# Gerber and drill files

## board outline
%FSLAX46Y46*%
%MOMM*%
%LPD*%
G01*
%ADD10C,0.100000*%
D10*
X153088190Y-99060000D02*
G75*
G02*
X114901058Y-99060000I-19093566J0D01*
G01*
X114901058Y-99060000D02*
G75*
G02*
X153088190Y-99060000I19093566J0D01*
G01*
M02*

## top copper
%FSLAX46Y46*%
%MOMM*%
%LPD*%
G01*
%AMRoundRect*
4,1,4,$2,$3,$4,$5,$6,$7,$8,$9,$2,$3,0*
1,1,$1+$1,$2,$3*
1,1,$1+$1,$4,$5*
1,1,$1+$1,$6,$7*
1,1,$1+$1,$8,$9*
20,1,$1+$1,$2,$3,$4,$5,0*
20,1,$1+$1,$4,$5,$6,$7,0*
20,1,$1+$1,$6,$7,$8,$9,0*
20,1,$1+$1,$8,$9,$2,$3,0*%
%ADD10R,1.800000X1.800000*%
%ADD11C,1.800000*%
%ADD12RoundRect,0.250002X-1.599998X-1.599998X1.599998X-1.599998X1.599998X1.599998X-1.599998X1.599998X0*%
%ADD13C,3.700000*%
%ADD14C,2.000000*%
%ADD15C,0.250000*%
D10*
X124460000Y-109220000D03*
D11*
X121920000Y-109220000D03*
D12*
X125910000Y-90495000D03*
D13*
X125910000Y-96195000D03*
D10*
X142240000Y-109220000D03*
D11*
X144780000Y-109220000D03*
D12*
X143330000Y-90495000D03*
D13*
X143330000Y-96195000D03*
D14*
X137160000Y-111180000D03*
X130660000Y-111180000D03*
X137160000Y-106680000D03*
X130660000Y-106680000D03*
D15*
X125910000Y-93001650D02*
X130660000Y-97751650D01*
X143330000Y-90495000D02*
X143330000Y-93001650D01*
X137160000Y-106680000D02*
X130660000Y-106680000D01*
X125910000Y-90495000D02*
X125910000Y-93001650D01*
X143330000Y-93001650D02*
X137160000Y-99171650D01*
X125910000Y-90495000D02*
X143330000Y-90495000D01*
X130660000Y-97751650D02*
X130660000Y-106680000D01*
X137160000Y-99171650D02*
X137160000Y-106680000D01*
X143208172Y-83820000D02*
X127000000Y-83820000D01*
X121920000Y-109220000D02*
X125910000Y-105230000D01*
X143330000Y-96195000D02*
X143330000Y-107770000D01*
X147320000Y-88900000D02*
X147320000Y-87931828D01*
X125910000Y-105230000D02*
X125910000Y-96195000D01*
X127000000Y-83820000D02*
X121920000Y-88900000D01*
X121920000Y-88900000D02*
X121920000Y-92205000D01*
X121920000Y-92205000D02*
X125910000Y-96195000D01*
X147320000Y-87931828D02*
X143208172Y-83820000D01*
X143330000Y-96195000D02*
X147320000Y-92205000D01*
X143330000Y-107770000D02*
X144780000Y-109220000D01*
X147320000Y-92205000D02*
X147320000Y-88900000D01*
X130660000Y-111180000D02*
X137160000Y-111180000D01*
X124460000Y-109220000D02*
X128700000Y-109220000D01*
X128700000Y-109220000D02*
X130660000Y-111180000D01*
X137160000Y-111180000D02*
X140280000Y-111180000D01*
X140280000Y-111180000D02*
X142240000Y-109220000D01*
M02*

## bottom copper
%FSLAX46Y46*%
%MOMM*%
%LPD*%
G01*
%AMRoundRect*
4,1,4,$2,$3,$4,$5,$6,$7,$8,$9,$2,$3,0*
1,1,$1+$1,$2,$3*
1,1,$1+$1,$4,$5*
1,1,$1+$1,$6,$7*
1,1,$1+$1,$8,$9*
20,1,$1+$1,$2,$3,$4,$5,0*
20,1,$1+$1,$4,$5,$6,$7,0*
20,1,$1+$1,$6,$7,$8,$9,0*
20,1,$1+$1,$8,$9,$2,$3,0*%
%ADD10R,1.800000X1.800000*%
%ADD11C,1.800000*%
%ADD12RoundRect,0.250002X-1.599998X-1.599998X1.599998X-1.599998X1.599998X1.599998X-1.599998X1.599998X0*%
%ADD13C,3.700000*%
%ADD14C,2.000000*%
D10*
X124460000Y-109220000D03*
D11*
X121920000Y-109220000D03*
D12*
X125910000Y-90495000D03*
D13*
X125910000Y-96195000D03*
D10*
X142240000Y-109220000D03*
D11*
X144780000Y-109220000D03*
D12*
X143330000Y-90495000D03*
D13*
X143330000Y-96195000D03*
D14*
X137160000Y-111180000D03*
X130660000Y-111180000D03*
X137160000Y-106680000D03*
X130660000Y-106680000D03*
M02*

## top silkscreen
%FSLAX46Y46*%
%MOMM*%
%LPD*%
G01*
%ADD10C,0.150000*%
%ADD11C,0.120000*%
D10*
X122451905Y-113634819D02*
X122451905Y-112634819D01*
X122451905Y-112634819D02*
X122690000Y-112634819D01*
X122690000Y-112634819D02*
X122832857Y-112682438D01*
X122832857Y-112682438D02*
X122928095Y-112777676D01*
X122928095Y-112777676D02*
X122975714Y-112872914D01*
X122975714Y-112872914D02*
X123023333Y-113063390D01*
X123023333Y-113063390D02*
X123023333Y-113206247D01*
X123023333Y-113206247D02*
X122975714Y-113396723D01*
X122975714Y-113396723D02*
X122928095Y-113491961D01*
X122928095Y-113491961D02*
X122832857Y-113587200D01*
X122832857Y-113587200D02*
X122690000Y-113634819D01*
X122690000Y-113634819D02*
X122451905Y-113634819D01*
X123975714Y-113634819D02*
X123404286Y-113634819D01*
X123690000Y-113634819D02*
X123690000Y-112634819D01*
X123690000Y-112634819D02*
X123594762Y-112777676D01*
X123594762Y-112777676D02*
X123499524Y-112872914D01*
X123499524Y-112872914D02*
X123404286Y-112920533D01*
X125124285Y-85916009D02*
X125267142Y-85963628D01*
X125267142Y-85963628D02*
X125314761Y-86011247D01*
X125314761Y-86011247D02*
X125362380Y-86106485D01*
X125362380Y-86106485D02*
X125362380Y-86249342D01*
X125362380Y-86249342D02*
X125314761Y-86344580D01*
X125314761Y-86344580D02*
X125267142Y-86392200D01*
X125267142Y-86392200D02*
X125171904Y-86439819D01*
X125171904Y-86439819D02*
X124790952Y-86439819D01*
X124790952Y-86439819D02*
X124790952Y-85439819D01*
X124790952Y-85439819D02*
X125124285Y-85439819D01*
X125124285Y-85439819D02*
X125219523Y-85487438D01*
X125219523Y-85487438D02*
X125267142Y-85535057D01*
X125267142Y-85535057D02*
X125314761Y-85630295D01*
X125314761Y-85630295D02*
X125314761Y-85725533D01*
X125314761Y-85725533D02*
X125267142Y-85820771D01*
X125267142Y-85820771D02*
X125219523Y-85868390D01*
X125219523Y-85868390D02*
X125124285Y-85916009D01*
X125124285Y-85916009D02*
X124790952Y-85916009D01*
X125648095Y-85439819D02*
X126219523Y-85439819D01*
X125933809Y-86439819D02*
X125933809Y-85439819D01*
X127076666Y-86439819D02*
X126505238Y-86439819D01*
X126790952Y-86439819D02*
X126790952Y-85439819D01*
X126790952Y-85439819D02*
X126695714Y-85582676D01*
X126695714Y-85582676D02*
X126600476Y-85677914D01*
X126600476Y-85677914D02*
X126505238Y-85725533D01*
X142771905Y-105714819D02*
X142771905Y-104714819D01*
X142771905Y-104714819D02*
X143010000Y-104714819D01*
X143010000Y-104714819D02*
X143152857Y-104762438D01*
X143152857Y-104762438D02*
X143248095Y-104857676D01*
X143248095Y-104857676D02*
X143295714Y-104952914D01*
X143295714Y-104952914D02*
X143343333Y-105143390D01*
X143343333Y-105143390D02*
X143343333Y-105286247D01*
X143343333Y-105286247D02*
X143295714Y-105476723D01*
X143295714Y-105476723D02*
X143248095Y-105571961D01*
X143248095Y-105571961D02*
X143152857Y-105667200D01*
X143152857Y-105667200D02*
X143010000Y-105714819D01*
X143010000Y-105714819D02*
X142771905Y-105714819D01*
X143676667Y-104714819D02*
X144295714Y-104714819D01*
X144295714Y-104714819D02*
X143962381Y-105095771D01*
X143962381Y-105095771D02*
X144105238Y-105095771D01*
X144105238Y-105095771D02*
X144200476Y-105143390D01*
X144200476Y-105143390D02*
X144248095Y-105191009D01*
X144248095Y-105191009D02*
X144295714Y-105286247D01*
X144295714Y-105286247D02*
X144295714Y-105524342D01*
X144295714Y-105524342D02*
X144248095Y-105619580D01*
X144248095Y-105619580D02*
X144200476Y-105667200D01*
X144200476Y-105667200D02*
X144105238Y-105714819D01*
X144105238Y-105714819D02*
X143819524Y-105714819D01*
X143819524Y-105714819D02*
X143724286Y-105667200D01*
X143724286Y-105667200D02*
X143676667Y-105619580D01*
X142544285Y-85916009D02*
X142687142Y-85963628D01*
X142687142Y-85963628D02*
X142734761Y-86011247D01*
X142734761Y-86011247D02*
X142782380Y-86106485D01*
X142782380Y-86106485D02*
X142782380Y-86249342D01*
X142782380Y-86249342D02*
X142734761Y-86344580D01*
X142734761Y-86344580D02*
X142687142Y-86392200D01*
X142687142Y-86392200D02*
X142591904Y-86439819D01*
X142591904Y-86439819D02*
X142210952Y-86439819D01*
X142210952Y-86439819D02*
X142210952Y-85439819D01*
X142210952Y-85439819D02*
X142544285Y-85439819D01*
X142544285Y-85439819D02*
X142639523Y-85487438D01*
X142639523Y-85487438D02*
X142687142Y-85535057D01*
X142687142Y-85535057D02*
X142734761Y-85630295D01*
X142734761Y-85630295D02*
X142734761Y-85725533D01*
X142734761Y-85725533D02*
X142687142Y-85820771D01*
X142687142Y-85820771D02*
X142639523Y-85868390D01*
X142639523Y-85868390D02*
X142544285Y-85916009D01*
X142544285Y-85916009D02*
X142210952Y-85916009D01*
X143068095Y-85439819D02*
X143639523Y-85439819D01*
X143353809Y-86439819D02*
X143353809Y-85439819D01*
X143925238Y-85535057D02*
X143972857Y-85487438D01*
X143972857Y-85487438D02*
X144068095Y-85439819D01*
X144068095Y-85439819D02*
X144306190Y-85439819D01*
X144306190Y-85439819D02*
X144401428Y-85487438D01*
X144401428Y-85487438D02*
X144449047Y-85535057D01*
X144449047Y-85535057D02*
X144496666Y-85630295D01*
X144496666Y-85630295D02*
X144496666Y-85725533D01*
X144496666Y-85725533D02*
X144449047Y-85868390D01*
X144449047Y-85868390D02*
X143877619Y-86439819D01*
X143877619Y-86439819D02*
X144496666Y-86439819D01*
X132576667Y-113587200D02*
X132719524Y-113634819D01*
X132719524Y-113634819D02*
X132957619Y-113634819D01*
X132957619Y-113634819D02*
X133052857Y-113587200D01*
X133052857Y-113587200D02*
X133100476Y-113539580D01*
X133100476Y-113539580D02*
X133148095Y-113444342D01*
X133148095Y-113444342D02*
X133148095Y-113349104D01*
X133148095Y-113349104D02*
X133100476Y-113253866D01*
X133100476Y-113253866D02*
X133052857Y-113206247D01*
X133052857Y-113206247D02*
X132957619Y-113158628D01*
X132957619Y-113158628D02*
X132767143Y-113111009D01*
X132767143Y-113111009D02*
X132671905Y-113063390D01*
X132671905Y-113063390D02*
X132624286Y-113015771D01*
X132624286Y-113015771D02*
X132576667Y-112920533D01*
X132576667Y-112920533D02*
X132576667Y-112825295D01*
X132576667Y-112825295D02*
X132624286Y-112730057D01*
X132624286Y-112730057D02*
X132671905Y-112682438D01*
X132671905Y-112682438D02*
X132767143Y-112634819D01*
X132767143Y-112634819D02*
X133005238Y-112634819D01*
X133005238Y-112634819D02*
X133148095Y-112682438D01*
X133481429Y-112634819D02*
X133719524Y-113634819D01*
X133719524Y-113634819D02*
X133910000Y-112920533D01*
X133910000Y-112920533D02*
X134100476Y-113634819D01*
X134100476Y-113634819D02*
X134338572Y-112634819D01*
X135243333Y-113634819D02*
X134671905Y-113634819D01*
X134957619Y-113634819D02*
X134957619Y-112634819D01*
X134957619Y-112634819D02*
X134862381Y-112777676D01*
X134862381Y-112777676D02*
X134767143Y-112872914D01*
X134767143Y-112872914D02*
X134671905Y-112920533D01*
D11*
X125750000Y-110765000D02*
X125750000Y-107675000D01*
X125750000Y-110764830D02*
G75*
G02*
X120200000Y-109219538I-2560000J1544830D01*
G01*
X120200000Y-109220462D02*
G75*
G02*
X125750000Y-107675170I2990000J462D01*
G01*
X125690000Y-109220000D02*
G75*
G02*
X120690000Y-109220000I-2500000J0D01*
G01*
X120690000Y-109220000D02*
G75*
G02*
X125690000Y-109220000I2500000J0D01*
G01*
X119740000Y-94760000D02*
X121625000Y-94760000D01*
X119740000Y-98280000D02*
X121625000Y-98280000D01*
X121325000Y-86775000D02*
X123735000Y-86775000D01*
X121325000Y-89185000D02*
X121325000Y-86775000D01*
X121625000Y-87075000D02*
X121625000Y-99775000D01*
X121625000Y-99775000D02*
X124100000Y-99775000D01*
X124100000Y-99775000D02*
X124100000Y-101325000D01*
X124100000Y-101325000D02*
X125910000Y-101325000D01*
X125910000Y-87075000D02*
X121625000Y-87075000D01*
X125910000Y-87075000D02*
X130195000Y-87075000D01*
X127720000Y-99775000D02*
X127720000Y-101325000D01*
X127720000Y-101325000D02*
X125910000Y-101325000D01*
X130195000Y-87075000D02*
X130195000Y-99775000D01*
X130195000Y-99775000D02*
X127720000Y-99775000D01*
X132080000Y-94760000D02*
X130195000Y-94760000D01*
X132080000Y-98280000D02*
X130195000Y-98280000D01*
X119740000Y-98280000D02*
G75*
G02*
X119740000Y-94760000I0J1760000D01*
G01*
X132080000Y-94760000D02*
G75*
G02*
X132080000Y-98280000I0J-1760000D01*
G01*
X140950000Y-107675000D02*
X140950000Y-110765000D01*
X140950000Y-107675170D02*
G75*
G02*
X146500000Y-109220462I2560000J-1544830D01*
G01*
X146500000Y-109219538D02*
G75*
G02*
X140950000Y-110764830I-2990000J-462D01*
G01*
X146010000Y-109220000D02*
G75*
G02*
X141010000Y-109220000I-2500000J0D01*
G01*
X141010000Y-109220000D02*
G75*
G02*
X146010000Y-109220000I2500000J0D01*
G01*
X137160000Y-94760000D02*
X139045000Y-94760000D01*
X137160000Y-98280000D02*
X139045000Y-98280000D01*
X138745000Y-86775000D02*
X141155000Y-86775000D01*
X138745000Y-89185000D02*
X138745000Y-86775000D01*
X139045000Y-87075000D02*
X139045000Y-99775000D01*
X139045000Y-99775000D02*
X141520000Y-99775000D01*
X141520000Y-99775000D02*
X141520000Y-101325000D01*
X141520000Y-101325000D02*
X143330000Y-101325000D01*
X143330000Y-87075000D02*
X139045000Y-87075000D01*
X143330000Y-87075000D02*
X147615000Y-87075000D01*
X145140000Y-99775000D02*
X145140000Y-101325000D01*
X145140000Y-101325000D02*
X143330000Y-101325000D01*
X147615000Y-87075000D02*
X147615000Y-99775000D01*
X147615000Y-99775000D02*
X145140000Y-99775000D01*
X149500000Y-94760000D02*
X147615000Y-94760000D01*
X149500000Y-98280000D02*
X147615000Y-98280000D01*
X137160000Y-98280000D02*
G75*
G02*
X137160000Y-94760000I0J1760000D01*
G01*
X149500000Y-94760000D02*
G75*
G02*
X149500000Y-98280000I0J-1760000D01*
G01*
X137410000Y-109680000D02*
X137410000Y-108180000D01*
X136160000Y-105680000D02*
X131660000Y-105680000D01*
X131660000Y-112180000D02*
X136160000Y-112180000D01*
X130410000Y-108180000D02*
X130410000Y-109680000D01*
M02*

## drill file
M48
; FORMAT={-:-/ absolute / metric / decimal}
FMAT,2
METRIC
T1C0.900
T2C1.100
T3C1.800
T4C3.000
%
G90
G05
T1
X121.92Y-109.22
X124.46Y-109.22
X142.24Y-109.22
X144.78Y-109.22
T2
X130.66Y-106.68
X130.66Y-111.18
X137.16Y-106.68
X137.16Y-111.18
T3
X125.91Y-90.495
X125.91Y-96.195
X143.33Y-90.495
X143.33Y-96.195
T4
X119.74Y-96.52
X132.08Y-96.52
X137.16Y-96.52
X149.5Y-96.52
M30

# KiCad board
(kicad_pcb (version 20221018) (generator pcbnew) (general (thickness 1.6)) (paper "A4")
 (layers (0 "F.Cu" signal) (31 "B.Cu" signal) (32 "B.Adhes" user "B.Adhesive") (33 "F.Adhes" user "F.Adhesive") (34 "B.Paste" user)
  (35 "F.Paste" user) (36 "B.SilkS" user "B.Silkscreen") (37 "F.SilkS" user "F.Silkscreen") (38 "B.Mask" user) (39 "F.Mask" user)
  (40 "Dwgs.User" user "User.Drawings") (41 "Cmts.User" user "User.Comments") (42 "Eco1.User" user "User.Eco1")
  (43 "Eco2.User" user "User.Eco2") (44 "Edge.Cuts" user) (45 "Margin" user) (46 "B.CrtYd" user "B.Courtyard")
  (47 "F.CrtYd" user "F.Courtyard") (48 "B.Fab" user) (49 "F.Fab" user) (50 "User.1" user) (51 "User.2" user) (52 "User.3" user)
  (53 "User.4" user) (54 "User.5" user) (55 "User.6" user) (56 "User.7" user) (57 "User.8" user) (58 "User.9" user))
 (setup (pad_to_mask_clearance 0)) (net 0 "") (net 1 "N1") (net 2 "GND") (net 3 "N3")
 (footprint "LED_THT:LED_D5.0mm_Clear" (layer "F.Cu") (at 124.46 109.22 180)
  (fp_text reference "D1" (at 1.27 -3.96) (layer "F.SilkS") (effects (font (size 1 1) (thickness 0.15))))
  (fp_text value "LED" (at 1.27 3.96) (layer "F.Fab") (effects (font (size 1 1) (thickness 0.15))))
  (fp_line (start -1.29 -1.545) (end -1.29 1.545) (stroke (width 0.12) (type solid)) (layer "F.SilkS"))
  (fp_arc (start -1.29 -1.54483) (mid 2.072002 -2.880433) (end 4.26 0.000462) (stroke (width 0.12) (type solid)) (layer "F.SilkS"))
  (fp_arc (start 4.26 -0.000462) (mid 2.072002 2.880433) (end -1.29 1.54483) (stroke (width 0.12) (type solid)) (layer "F.SilkS"))
  (fp_circle (center 1.27 0) (end 3.77 0) (stroke (width 0.12) (type solid)) (fill none) (layer "F.SilkS"))
  (pad "1" thru_hole rect (at 0 0 180) (size 1.8 1.8) (drill 0.9) (layers "*.Cu" "*.Mask") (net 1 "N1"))
  (pad "2" thru_hole circle (at 2.54 0 180) (size 1.8 1.8) (drill 0.9) (layers "*.Cu" "*.Mask") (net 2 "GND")))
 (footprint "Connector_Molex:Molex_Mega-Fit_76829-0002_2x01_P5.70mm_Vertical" (layer "F.Cu") (at 125.91 90.495)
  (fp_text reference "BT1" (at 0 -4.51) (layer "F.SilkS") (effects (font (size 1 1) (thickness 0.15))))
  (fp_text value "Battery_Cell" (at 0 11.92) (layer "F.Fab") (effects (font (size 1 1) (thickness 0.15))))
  (fp_line (start -6.17 4.265) (end -4.285 4.265) (stroke (width 0.12) (type solid)) (layer "F.SilkS"))
  (fp_line (start -6.17 7.785) (end -4.285 7.785) (stroke (width 0.12) (type solid)) (layer "F.SilkS"))
  (fp_line (start -4.585 -3.72) (end -2.175 -3.72) (stroke (width 0.12) (type solid)) (layer "F.SilkS"))
  (fp_line (start -4.585 -1.31) (end -4.585 -3.72) (stroke (width 0.12) (type solid)) (layer "F.SilkS"))
  (fp_line (start -4.285 -3.42) (end -4.285 9.28) (stroke (width 0.12) (type solid)) (layer "F.SilkS"))
  (fp_line (start -4.285 9.28) (end -1.81 9.28) (stroke (width 0.12) (type solid)) (layer "F.SilkS"))
  (fp_line (start -1.81 9.28) (end -1.81 10.83) (stroke (width 0.12) (type solid)) (layer "F.SilkS"))
  (fp_line (start -1.81 10.83) (end 0 10.83) (stroke (width 0.12) (type solid)) (layer "F.SilkS"))
  (fp_line (start 0 -3.42) (end -4.285 -3.42) (stroke (width 0.12) (type solid)) (layer "F.SilkS"))
  (fp_line (start 0 -3.42) (end 4.285 -3.42) (stroke (width 0.12) (type solid)) (layer "F.SilkS"))
  (fp_line (start 1.81 9.28) (end 1.81 10.83) (stroke (width 0.12) (type solid)) (layer "F.SilkS"))
  (fp_line (start 1.81 10.83) (end 0 10.83) (stroke (width 0.12) (type solid)) (layer "F.SilkS"))
  (fp_line (start 4.285 -3.42) (end 4.285 9.28) (stroke (width 0.12) (type solid)) (layer "F.SilkS"))
  (fp_line (start 4.285 9.28) (end 1.81 9.28) (stroke (width 0.12) (type solid)) (layer "F.SilkS"))
  (fp_line (start 6.17 4.265) (end 4.285 4.265) (stroke (width 0.12) (type solid)) (layer "F.SilkS"))
  (fp_line (start 6.17 7.785) (end 4.285 7.785) (stroke (width 0.12) (type solid)) (layer "F.SilkS"))
  (fp_arc (start -6.17 7.785) (mid -7.93 6.025) (end -6.17 4.265) (stroke (width 0.12) (type solid)) (layer "F.SilkS"))
  (fp_arc (start 6.17 4.265) (mid 7.93 6.025) (end 6.17 7.785) (stroke (width 0.12) (type solid)) (layer "F.SilkS"))
  (pad "" np_thru_hole circle (at -6.17 6.025) (size 3 3) (drill 3) (layers "*.Cu" "*.Mask"))
  (pad "" np_thru_hole circle (at 6.17 6.025) (size 3 3) (drill 3) (layers "*.Cu" "*.Mask"))
  (pad "1" thru_hole roundrect (at 0 0) (size 3.7 3.7) (drill 1.8) (layers "*.Cu" "*.Mask") (roundrect_rratio 0.067568) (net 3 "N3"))
  (pad "2" thru_hole circle (at 0 5.7) (size 3.7 3.7) (drill 1.8) (layers "*.Cu" "*.Mask") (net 2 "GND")))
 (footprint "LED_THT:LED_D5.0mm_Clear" (layer "F.Cu") (at 142.24 109.22)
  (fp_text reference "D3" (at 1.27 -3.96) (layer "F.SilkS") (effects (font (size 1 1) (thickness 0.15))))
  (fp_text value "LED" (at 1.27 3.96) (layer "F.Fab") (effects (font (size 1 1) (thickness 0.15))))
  (fp_line (start -1.29 -1.545) (end -1.29 1.545) (stroke (width 0.12) (type solid)) (layer "F.SilkS"))
  (fp_arc (start -1.29 -1.54483) (mid 2.072002 -2.880433) (end 4.26 0.000462) (stroke (width 0.12) (type solid)) (layer "F.SilkS"))
  (fp_arc (start 4.26 -0.000462) (mid 2.072002 2.880433) (end -1.29 1.54483) (stroke (width 0.12) (type solid)) (layer "F.SilkS"))
  (fp_circle (center 1.27 0) (end 3.77 0) (stroke (width 0.12) (type solid)) (fill none) (layer "F.SilkS"))
  (pad "1" thru_hole rect (at 0 0) (size 1.8 1.8) (drill 0.9) (layers "*.Cu" "*.Mask") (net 1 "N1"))
  (pad "2" thru_hole circle (at 2.54 0) (size 1.8 1.8) (drill 0.9) (layers "*.Cu" "*.Mask") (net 2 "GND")))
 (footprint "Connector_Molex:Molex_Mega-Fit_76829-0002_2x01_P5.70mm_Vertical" (layer "F.Cu") (at 143.33 90.495)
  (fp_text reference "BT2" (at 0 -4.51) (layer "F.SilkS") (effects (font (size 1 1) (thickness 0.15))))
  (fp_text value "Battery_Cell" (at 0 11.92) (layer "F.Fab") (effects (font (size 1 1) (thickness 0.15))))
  (fp_line (start -6.17 4.265) (end -4.285 4.265) (stroke (width 0.12) (type solid)) (layer "F.SilkS"))
  (fp_line (start -6.17 7.785) (end -4.285 7.785) (stroke (width 0.12) (type solid)) (layer "F.SilkS"))
  (fp_line (start -4.585 -3.72) (end -2.175 -3.72) (stroke (width 0.12) (type solid)) (layer "F.SilkS"))
  (fp_line (start -4.585 -1.31) (end -4.585 -3.72) (stroke (width 0.12) (type solid)) (layer "F.SilkS"))
  (fp_line (start -4.285 -3.42) (end -4.285 9.28) (stroke (width 0.12) (type solid)) (layer "F.SilkS"))
  (fp_line (start -4.285 9.28) (end -1.81 9.28) (stroke (width 0.12) (type solid)) (layer "F.SilkS"))
  (fp_line (start -1.81 9.28) (end -1.81 10.83) (stroke (width 0.12) (type solid)) (layer "F.SilkS"))
  (fp_line (start -1.81 10.83) (end 0 10.83) (stroke (width 0.12) (type solid)) (layer "F.SilkS"))
  (fp_line (start 0 -3.42) (end -4.285 -3.42) (stroke (width 0.12) (type solid)) (layer "F.SilkS"))
  (fp_line (start 0 -3.42) (end 4.285 -3.42) (stroke (width 0.12) (type solid)) (layer "F.SilkS"))
  (fp_line (start 1.81 9.28) (end 1.81 10.83) (stroke (width 0.12) (type solid)) (layer "F.SilkS"))
  (fp_line (start 1.81 10.83) (end 0 10.83) (stroke (width 0.12) (type solid)) (layer "F.SilkS"))
  (fp_line (start 4.285 -3.42) (end 4.285 9.28) (stroke (width 0.12) (type solid)) (layer "F.SilkS"))
  (fp_line (start 4.285 9.28) (end 1.81 9.28) (stroke (width 0.12) (type solid)) (layer "F.SilkS"))
  (fp_line (start 6.17 4.265) (end 4.285 4.265) (stroke (width 0.12) (type solid)) (layer "F.SilkS"))
  (fp_line (start 6.17 7.785) (end 4.285 7.785) (stroke (width 0.12) (type solid)) (layer "F.SilkS"))
  (fp_arc (start -6.17 7.785) (mid -7.93 6.025) (end -6.17 4.265) (stroke (width 0.12) (type solid)) (layer "F.SilkS"))
  (fp_arc (start 6.17 4.265) (mid 7.93 6.025) (end 6.17 7.785) (stroke (width 0.12) (type solid)) (layer "F.SilkS"))
  (pad "" np_thru_hole circle (at -6.17 6.025) (size 3 3) (drill 3) (layers "*.Cu" "*.Mask"))
  (pad "" np_thru_hole circle (at 6.17 6.025) (size 3 3) (drill 3) (layers "*.Cu" "*.Mask"))
  (pad "1" thru_hole roundrect (at 0 0) (size 3.7 3.7) (drill 1.8) (layers "*.Cu" "*.Mask") (roundrect_rratio 0.067568) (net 3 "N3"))
  (pad "2" thru_hole circle (at 0 5.7) (size 3.7 3.7) (drill 1.8) (layers "*.Cu" "*.Mask") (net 2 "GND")))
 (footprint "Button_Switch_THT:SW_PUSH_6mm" (layer "F.Cu") (at 137.16 111.18 180)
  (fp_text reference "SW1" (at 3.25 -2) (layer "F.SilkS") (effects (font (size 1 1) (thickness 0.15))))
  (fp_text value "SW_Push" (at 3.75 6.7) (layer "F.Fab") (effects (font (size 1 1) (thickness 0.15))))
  (fp_line (start -0.25 1.5) (end -0.25 3) (stroke (width 0.12) (type solid)) (layer "F.SilkS"))
  (fp_line (start 1 5.5) (end 5.5 5.5) (stroke (width 0.12) (type solid)) (layer "F.SilkS"))
  (fp_line (start 5.5 -1) (end 1 -1) (stroke (width 0.12) (type solid)) (layer "F.SilkS"))
  (fp_line (start 6.75 3) (end 6.75 1.5) (stroke (width 0.12) (type solid)) (layer "F.SilkS"))
  (pad "1" thru_hole circle (at 0 0 270) (size 2 2) (drill 1.1) (layers "*.Cu" "*.Mask") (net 1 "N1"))
  (pad "1" thru_hole circle (at 6.5 0 270) (size 2 2) (drill 1.1) (layers "*.Cu" "*.Mask") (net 1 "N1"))
  (pad "2" thru_hole circle (at 0 4.5 270) (size 2 2) (drill 1.1) (layers "*.Cu" "*.Mask") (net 3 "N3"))
  (pad "2" thru_hole circle (at 6.5 4.5 270) (size 2 2) (drill 1.1) (layers "*.Cu" "*.Mask") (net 3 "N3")))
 (gr_circle (center 133.994624 99.06) (end 152.4 104.14) (stroke (width 0.1) (type default)) (fill none) (layer "Edge.Cuts"))
 (segment (start 125.91 93.00165) (end 130.66 97.75165) (width 0.25) (layer "F.Cu") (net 3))
 (segment (start 143.33 90.495) (end 143.33 93.00165) (width 0.25) (layer "F.Cu") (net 3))
 (segment (start 137.16 106.68) (end 130.66 106.68) (width 0.25) (layer "F.Cu") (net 3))
 (segment (start 125.91 90.495) (end 125.91 93.00165) (width 0.25) (layer "F.Cu") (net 3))
 (segment (start 143.33 93.00165) (end 137.16 99.17165) (width 0.25) (layer "F.Cu") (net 3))
 (segment (start 125.91 90.495) (end 143.33 90.495) (width 0.25) (layer "F.Cu") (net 3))
 (segment (start 130.66 97.75165) (end 130.66 106.68) (width 0.25) (layer "F.Cu") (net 3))
 (segment (start 137.16 99.17165) (end 137.16 106.68) (width 0.25) (layer "F.Cu") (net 3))
 (segment (start 143.208172 83.82) (end 127 83.82) (width 0.25) (layer "F.Cu") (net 2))
 (segment (start 121.92 109.22) (end 125.91 105.23) (width 0.25) (layer "F.Cu") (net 2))
 (segment (start 143.33 96.195) (end 143.33 107.77) (width 0.25) (layer "F.Cu") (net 2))
 (segment (start 147.32 88.9) (end 147.32 87.931828) (width 0.25) (layer "F.Cu") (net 2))
 (segment (start 125.91 105.23) (end 125.91 96.195) (width 0.25) (layer "F.Cu") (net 2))
 (segment (start 127 83.82) (end 121.92 88.9) (width 0.25) (layer "F.Cu") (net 2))
 (segment (start 121.92 88.9) (end 121.92 92.205) (width 0.25) (layer "F.Cu") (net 2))
 (segment (start 121.92 92.205) (end 125.91 96.195) (width 0.25) (layer "F.Cu") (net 2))
 (segment (start 147.32 87.931828) (end 143.208172 83.82) (width 0.25) (layer "F.Cu") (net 2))
 (segment (start 143.33 96.195) (end 147.32 92.205) (width 0.25) (layer "F.Cu") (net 2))
 (segment (start 143.33 107.77) (end 144.78 109.22) (width 0.25) (layer "F.Cu") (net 2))
 (segment (start 147.32 92.205) (end 147.32 88.9) (width 0.25) (layer "F.Cu") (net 2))
 (segment (start 130.66 111.18) (end 137.16 111.18) (width 0.25) (layer "F.Cu") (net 1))
 (segment (start 124.46 109.22) (end 128.7 109.22) (width 0.25) (layer "F.Cu") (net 1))
 (segment (start 128.7 109.22) (end 130.66 111.18) (width 0.25) (layer "F.Cu") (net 1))
 (segment (start 137.16 111.18) (end 140.28 111.18) (width 0.25) (layer "F.Cu") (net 1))
 (segment (start 140.28 111.18) (end 142.24 109.22) (width 0.25) (layer "F.Cu") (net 1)))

